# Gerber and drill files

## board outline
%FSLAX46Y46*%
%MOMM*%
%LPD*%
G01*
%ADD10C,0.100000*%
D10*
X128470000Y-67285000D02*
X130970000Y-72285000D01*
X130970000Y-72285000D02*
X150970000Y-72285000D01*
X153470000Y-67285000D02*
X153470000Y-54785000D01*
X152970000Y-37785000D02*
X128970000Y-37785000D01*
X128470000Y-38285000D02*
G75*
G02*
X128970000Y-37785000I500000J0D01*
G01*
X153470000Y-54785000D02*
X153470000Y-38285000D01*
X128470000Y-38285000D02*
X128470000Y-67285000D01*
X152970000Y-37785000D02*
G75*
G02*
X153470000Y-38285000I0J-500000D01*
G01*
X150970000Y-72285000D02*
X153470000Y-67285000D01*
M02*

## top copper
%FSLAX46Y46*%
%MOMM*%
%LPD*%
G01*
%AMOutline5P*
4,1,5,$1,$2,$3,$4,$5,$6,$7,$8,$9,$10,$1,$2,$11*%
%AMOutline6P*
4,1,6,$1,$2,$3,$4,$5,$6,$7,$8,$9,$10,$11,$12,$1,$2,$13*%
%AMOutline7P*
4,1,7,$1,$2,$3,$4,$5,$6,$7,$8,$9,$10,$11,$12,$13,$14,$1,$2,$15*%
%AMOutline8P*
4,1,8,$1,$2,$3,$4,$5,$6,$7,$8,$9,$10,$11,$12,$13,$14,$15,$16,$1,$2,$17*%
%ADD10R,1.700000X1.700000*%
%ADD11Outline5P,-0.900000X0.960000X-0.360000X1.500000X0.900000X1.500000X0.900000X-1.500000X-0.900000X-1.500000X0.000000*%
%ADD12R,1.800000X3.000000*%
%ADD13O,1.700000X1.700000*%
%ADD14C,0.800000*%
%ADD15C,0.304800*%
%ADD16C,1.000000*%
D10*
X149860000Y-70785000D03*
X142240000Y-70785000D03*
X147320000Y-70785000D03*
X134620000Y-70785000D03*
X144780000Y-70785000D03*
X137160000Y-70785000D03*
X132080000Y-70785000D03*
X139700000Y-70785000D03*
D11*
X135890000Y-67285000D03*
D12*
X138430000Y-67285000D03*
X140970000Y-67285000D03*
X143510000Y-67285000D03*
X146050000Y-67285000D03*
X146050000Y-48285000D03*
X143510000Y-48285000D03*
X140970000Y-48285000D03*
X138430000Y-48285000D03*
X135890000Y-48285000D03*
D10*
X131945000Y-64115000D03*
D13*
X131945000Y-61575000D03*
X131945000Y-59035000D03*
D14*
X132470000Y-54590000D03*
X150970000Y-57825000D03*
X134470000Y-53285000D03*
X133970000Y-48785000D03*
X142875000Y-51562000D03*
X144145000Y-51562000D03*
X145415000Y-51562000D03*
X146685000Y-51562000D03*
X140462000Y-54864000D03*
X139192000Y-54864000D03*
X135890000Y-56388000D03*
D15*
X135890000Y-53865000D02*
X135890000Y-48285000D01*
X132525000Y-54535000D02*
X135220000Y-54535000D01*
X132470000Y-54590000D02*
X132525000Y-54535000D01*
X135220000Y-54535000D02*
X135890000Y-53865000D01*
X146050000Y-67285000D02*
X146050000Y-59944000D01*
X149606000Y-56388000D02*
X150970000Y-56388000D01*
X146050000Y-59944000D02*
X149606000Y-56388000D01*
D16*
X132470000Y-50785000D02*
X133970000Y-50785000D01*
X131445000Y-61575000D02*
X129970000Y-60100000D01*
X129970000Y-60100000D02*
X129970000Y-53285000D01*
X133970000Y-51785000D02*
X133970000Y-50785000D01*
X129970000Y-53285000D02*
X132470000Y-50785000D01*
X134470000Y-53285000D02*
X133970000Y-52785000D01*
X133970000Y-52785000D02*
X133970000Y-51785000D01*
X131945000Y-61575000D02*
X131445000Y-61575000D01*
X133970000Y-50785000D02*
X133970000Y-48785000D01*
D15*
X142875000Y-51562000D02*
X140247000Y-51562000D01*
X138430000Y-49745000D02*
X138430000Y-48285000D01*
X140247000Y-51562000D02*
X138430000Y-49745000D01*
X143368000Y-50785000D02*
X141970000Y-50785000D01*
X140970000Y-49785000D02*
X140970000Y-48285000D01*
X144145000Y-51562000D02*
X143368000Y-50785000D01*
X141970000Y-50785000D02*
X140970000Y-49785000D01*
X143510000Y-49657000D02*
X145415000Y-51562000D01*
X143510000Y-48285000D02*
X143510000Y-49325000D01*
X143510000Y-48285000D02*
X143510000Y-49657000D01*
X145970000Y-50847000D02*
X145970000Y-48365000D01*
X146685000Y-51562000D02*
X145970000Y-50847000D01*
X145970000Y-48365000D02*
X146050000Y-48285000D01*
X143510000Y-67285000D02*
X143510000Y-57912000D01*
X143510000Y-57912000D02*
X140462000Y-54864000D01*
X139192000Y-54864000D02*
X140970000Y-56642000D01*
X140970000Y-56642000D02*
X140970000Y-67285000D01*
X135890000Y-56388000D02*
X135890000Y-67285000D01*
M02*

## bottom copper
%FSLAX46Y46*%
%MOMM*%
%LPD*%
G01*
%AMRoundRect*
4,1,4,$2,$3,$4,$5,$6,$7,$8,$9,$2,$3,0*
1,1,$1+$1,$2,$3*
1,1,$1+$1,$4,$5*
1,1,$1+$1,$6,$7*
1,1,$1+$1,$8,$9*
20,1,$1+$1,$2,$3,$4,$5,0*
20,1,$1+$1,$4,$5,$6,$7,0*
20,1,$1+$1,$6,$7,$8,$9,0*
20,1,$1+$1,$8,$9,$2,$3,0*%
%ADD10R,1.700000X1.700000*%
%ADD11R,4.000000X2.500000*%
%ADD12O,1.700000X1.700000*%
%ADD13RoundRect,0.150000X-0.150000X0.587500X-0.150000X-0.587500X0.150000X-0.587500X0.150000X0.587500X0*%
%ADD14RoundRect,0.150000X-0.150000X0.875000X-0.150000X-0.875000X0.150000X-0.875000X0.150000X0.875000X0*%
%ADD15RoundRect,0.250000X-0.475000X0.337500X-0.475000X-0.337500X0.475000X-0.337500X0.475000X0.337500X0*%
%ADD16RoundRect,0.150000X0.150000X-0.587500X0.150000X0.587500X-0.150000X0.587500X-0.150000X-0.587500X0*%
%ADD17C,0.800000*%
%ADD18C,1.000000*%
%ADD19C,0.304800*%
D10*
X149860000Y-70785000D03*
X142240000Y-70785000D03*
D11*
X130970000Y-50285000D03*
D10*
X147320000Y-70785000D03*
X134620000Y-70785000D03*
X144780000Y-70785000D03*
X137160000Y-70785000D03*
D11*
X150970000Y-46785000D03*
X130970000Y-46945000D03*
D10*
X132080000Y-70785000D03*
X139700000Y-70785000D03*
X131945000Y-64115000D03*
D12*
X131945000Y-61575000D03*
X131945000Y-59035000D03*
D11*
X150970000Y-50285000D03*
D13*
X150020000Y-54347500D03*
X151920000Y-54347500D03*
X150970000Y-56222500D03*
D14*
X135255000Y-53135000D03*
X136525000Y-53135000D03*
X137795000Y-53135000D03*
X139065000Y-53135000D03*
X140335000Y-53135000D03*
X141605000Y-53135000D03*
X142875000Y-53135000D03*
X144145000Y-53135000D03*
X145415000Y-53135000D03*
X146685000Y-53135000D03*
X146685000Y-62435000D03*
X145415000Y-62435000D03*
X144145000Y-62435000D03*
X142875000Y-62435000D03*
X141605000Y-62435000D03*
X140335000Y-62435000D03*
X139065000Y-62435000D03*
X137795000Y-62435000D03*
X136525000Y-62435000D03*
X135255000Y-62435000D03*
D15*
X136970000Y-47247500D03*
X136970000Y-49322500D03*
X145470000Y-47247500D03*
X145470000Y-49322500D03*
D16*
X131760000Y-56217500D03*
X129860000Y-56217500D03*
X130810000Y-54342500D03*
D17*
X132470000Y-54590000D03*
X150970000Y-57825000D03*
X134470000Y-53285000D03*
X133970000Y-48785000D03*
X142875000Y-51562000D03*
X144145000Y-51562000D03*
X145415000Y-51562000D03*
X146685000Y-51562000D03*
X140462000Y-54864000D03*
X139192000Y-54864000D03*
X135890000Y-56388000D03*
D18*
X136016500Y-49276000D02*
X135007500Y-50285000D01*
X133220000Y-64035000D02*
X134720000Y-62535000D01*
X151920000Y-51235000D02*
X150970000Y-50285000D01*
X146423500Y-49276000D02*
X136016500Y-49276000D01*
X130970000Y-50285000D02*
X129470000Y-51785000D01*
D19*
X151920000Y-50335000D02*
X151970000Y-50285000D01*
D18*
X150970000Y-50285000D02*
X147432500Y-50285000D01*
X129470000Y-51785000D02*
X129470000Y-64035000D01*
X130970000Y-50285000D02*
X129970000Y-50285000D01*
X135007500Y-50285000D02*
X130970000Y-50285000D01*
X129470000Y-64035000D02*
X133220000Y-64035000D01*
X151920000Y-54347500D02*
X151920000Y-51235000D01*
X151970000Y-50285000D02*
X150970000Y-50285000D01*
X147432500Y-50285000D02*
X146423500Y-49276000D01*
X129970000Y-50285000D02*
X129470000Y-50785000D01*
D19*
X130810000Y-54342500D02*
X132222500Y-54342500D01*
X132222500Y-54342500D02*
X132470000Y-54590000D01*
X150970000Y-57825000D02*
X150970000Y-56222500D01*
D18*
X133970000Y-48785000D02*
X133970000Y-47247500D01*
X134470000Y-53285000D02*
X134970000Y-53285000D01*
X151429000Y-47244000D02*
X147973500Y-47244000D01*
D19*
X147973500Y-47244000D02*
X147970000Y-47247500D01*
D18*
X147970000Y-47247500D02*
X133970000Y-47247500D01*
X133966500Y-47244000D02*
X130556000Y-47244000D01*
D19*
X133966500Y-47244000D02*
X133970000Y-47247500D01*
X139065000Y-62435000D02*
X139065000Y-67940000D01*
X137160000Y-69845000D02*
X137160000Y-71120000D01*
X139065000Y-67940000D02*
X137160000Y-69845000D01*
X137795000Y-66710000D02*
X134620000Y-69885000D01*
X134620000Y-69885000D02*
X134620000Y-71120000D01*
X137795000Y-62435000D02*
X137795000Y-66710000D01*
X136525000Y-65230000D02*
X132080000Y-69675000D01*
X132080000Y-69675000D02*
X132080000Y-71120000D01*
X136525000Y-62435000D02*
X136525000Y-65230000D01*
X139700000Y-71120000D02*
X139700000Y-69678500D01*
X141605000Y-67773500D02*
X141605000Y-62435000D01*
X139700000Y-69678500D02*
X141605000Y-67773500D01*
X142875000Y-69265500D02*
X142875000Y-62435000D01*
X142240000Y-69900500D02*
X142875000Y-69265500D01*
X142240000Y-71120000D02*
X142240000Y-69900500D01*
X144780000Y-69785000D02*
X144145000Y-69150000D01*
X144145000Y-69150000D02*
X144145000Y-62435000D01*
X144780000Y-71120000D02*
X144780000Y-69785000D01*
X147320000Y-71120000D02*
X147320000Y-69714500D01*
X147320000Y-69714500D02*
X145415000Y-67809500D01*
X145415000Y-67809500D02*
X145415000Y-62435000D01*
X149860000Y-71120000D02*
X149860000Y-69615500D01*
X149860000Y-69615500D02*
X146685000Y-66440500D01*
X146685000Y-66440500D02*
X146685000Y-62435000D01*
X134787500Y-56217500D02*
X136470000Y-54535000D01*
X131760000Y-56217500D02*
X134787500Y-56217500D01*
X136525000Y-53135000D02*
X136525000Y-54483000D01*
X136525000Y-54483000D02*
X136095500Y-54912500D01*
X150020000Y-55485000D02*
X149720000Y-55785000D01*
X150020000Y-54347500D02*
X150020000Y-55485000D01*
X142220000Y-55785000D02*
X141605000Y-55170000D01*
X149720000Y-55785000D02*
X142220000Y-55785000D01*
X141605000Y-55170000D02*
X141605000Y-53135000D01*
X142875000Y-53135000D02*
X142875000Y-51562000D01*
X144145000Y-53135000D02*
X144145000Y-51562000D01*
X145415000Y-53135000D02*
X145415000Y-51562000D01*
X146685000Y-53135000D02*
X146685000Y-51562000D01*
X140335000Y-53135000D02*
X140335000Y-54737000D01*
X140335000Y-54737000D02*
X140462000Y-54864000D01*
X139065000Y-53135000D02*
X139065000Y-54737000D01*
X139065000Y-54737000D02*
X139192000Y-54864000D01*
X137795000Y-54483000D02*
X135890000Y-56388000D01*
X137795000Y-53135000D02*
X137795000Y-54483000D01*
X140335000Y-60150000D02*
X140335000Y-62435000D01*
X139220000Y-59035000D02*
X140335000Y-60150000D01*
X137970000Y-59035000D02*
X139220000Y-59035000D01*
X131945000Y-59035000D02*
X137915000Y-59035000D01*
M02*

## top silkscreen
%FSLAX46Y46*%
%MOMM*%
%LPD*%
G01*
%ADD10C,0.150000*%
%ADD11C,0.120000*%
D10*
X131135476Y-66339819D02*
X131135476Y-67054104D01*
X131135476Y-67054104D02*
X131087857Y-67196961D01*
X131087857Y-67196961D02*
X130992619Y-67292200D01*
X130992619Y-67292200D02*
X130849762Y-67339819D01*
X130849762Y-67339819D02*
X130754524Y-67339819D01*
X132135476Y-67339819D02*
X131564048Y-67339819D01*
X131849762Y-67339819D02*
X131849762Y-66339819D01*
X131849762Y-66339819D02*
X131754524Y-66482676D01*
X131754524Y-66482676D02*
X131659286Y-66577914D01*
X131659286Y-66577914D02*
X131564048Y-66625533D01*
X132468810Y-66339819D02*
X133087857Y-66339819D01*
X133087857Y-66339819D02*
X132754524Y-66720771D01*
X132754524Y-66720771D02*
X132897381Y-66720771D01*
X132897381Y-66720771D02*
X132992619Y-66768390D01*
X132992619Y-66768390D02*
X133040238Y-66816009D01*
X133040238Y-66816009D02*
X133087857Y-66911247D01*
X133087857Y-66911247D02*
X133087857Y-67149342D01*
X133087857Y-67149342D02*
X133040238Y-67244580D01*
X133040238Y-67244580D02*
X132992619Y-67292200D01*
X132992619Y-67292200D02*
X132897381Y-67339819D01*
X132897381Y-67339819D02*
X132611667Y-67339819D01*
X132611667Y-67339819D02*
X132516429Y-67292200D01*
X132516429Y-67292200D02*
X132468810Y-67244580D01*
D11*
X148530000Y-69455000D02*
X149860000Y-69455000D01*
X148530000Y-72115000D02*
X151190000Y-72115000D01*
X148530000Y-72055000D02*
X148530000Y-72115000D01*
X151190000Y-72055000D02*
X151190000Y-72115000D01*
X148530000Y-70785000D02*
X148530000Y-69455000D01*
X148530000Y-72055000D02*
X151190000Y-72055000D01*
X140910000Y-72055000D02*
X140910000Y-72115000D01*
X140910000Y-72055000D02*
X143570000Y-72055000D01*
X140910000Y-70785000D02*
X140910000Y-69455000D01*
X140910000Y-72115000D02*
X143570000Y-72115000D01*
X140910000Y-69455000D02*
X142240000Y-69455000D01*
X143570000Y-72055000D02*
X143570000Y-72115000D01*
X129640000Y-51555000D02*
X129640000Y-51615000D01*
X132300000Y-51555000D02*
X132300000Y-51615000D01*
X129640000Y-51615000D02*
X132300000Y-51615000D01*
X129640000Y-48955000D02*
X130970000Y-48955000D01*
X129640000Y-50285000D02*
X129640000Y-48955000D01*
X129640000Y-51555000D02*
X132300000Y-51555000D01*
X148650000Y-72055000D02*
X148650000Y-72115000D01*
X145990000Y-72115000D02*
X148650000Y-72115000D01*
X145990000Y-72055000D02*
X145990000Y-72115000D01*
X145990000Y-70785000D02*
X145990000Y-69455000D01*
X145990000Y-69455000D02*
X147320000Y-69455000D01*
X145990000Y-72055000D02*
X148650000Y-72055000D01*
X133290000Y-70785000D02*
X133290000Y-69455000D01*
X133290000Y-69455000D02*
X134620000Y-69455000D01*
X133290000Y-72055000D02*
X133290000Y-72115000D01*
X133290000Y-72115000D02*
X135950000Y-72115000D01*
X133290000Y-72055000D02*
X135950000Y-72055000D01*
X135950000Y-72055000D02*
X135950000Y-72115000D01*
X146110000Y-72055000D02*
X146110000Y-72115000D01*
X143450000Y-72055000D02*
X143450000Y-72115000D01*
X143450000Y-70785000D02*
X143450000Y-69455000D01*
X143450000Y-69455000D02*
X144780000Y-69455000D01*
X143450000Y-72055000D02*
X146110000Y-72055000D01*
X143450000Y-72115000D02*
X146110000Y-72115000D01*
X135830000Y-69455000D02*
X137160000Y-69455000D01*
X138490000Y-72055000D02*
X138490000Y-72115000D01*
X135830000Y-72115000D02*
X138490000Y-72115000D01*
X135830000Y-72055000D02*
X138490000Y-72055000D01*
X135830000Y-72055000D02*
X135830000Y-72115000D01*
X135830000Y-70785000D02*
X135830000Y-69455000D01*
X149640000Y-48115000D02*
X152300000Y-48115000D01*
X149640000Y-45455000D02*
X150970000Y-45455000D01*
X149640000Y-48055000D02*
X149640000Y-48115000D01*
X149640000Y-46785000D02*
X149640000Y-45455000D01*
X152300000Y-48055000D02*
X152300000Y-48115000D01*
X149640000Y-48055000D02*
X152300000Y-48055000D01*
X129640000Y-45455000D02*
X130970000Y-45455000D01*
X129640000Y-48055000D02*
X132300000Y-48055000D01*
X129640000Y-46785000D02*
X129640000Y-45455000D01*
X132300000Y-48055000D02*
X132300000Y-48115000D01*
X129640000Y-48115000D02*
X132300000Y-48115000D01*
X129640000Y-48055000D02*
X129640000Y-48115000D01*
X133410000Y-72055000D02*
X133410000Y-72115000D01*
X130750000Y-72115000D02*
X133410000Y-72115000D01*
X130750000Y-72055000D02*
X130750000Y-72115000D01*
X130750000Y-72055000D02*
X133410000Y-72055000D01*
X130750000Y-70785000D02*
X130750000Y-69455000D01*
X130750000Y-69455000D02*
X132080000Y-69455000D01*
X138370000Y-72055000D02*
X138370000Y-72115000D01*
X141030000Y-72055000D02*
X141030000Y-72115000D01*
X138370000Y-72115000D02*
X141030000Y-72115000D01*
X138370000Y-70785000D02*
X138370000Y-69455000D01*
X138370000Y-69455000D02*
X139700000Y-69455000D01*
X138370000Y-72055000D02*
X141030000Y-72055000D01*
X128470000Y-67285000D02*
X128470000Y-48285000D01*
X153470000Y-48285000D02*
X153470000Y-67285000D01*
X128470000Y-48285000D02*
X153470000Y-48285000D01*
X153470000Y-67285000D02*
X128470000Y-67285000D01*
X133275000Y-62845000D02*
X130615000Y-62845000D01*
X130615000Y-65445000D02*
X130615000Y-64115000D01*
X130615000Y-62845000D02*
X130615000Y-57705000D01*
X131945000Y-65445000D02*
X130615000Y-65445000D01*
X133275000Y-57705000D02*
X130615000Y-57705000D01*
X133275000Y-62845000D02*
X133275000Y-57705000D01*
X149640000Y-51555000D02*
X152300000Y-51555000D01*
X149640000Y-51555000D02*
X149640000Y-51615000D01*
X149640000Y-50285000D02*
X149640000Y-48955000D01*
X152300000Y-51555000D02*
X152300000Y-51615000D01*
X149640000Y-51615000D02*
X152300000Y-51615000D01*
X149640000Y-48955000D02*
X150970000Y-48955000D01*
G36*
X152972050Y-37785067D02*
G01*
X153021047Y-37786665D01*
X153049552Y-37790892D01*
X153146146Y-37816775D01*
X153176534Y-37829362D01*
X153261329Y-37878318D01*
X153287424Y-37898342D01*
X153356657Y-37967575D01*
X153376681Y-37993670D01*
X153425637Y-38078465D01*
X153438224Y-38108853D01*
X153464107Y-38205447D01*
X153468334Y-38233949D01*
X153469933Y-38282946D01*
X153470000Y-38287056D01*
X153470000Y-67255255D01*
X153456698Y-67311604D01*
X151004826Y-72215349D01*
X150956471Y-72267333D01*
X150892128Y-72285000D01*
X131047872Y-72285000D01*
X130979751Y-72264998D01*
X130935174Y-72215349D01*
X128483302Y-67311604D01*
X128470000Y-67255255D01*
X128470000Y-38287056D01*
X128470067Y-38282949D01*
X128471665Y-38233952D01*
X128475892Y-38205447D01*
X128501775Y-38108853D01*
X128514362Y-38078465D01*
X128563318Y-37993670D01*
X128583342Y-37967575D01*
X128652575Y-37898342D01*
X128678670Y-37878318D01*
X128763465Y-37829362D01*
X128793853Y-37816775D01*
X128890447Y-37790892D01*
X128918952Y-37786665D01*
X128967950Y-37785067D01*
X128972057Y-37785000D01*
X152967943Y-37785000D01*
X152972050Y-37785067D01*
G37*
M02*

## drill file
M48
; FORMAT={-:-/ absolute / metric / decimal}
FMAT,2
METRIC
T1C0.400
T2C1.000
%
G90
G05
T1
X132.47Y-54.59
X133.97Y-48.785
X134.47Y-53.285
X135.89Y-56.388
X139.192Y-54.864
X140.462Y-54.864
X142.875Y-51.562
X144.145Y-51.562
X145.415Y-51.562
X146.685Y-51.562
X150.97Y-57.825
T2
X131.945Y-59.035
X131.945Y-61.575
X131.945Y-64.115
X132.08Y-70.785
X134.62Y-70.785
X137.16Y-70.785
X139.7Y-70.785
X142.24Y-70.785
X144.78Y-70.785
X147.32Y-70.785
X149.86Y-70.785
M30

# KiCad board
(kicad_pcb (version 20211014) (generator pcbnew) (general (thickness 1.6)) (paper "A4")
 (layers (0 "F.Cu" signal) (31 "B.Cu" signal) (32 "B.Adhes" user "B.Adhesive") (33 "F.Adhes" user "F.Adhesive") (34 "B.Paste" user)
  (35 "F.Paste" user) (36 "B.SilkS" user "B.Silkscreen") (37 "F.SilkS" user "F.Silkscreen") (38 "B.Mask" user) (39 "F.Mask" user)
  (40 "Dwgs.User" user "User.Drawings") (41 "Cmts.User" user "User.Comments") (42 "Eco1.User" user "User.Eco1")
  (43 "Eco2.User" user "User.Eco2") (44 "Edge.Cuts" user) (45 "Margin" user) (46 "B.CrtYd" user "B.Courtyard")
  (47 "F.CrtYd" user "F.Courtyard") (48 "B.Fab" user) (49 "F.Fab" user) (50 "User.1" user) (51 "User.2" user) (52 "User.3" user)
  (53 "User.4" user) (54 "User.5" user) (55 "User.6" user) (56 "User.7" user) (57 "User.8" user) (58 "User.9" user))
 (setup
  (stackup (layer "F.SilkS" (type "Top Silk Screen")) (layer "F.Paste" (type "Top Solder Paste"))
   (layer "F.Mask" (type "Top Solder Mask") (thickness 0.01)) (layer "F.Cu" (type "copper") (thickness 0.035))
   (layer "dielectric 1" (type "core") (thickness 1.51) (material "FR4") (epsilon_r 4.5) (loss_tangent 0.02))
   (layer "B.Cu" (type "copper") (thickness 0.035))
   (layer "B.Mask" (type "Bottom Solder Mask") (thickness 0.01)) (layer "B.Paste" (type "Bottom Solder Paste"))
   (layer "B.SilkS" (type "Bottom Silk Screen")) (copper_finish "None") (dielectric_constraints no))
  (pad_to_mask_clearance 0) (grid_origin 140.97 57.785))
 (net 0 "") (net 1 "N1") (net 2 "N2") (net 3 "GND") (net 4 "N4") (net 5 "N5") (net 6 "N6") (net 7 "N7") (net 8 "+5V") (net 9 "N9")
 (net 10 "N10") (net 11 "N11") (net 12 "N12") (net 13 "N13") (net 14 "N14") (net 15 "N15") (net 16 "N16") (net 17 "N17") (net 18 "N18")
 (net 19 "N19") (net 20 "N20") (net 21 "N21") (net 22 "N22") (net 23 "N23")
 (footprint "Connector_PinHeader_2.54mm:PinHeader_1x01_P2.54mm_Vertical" (layer "F.Cu") (at 149.86 70.785)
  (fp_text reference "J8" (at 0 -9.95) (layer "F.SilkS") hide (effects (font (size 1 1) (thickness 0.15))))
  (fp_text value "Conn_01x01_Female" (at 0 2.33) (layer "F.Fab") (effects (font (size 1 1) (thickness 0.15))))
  (fp_line (start -1.33 -1.33) (end 0 -1.33) (layer "F.SilkS") (width 0.12))
  (fp_line (start -1.33 1.33) (end 1.33 1.33) (layer "F.SilkS") (width 0.12))
  (fp_line (start -1.33 1.27) (end -1.33 1.33) (layer "F.SilkS") (width 0.12))
  (fp_line (start 1.33 1.27) (end 1.33 1.33) (layer "F.SilkS") (width 0.12))
  (fp_line (start -1.33 0) (end -1.33 -1.33) (layer "F.SilkS") (width 0.12))
  (fp_line (start -1.33 1.27) (end 1.33 1.27) (layer "F.SilkS") (width 0.12))
  (pad "1" thru_hole rect (at 0 0) (size 1.7 1.7) (drill 1) (layers *.Cu *.Mask) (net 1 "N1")))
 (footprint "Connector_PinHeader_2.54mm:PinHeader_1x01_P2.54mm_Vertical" (layer "F.Cu") (at 142.24 70.785)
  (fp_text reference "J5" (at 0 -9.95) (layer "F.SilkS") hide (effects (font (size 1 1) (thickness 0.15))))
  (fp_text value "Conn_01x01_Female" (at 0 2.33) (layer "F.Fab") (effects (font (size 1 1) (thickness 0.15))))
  (fp_line (start -1.33 1.27) (end -1.33 1.33) (layer "F.SilkS") (width 0.12))
  (fp_line (start -1.33 1.27) (end 1.33 1.27) (layer "F.SilkS") (width 0.12))
  (fp_line (start -1.33 0) (end -1.33 -1.33) (layer "F.SilkS") (width 0.12))
  (fp_line (start -1.33 1.33) (end 1.33 1.33) (layer "F.SilkS") (width 0.12))
  (fp_line (start -1.33 -1.33) (end 0 -1.33) (layer "F.SilkS") (width 0.12))
  (fp_line (start 1.33 1.27) (end 1.33 1.33) (layer "F.SilkS") (width 0.12))
  (pad "1" thru_hole rect (at 0 0) (size 1.7 1.7) (drill 1) (layers *.Cu *.Mask) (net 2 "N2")))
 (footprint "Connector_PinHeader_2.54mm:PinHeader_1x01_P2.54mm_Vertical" (layer "F.Cu") (at 130.97 50.285)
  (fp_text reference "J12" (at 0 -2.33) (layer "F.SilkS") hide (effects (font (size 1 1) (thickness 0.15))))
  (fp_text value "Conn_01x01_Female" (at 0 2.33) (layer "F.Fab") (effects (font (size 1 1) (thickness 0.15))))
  (fp_line (start -1.33 1.27) (end -1.33 1.33) (layer "F.SilkS") (width 0.12))
  (fp_line (start 1.33 1.27) (end 1.33 1.33) (layer "F.SilkS") (width 0.12))
  (fp_line (start -1.33 1.33) (end 1.33 1.33) (layer "F.SilkS") (width 0.12))
  (fp_line (start -1.33 -1.33) (end 0 -1.33) (layer "F.SilkS") (width 0.12))
  (fp_line (start -1.33 0) (end -1.33 -1.33) (layer "F.SilkS") (width 0.12))
  (fp_line (start -1.33 1.27) (end 1.33 1.27) (layer "F.SilkS") (width 0.12))
  (pad "1" smd rect (at 0 0) (size 4 2.5) (layers "B.Cu" "B.Mask") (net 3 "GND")))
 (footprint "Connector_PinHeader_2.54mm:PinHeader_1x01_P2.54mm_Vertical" (layer "F.Cu") (at 147.32 70.785)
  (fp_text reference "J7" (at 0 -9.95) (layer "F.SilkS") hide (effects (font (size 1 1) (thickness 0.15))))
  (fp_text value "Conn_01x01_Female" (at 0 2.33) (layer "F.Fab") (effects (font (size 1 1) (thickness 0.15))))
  (fp_line (start 1.33 1.27) (end 1.33 1.33) (layer "F.SilkS") (width 0.12))
  (fp_line (start -1.33 1.33) (end 1.33 1.33) (layer "F.SilkS") (width 0.12))
  (fp_line (start -1.33 1.27) (end -1.33 1.33) (layer "F.SilkS") (width 0.12))
  (fp_line (start -1.33 0) (end -1.33 -1.33) (layer "F.SilkS") (width 0.12))
  (fp_line (start -1.33 -1.33) (end 0 -1.33) (layer "F.SilkS") (width 0.12))
  (fp_line (start -1.33 1.27) (end 1.33 1.27) (layer "F.SilkS") (width 0.12))
  (pad "1" thru_hole rect (at 0 0) (size 1.7 1.7) (drill 1) (layers *.Cu *.Mask) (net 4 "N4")))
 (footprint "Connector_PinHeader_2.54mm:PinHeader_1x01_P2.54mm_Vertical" (layer "F.Cu") (at 134.62 70.785)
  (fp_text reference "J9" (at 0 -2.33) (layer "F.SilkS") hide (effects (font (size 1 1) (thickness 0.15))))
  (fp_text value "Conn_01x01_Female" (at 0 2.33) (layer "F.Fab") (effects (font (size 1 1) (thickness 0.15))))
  (fp_line (start -1.33 0) (end -1.33 -1.33) (layer "F.SilkS") (width 0.12))
  (fp_line (start -1.33 -1.33) (end 0 -1.33) (layer "F.SilkS") (width 0.12))
  (fp_line (start -1.33 1.27) (end -1.33 1.33) (layer "F.SilkS") (width 0.12))
  (fp_line (start -1.33 1.33) (end 1.33 1.33) (layer "F.SilkS") (width 0.12))
  (fp_line (start -1.33 1.27) (end 1.33 1.27) (layer "F.SilkS") (width 0.12))
  (fp_line (start 1.33 1.27) (end 1.33 1.33) (layer "F.SilkS") (width 0.12))
  (pad "1" thru_hole rect (at 0 0) (size 1.7 1.7) (drill 1) (layers *.Cu *.Mask) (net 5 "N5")))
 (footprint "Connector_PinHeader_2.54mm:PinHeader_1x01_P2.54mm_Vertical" (layer "F.Cu") (at 144.78 70.785)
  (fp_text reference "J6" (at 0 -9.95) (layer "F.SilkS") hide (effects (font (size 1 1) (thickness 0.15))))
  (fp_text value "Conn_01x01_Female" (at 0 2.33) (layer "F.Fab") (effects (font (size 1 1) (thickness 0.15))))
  (fp_line (start 1.33 1.27) (end 1.33 1.33) (layer "F.SilkS") (width 0.12))
  (fp_line (start -1.33 1.27) (end -1.33 1.33) (layer "F.SilkS") (width 0.12))
  (fp_line (start -1.33 0) (end -1.33 -1.33) (layer "F.SilkS") (width 0.12))
  (fp_line (start -1.33 -1.33) (end 0 -1.33) (layer "F.SilkS") (width 0.12))
  (fp_line (start -1.33 1.27) (end 1.33 1.27) (layer "F.SilkS") (width 0.12))
  (fp_line (start -1.33 1.33) (end 1.33 1.33) (layer "F.SilkS") (width 0.12))
  (pad "1" thru_hole rect (at 0 0) (size 1.7 1.7) (drill 1) (layers *.Cu *.Mask) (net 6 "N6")))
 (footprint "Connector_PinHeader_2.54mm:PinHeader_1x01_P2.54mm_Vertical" (layer "F.Cu") (at 137.16 70.785)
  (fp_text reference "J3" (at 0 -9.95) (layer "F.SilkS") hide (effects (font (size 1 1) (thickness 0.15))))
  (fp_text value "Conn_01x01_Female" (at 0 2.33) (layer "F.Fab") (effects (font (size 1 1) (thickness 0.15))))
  (fp_line (start -1.33 -1.33) (end 0 -1.33) (layer "F.SilkS") (width 0.12))
  (fp_line (start 1.33 1.27) (end 1.33 1.33) (layer "F.SilkS") (width 0.12))
  (fp_line (start -1.33 1.33) (end 1.33 1.33) (layer "F.SilkS") (width 0.12))
  (fp_line (start -1.33 1.27) (end 1.33 1.27) (layer "F.SilkS") (width 0.12))
  (fp_line (start -1.33 1.27) (end -1.33 1.33) (layer "F.SilkS") (width 0.12))
  (fp_line (start -1.33 0) (end -1.33 -1.33) (layer "F.SilkS") (width 0.12))
  (pad "1" thru_hole rect (at 0 0) (size 1.7 1.7) (drill 1) (layers *.Cu *.Mask) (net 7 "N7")))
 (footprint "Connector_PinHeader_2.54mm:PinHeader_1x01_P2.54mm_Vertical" (layer "F.Cu") (at 150.97 46.785)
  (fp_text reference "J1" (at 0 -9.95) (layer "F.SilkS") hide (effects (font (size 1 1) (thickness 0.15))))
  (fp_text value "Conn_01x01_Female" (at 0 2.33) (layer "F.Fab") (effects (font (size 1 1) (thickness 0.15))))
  (fp_line (start -1.33 1.33) (end 1.33 1.33) (layer "F.SilkS") (width 0.12))
  (fp_line (start -1.33 -1.33) (end 0 -1.33) (layer "F.SilkS") (width 0.12))
  (fp_line (start -1.33 1.27) (end -1.33 1.33) (layer "F.SilkS") (width 0.12))
  (fp_line (start -1.33 0) (end -1.33 -1.33) (layer "F.SilkS") (width 0.12))
  (fp_line (start 1.33 1.27) (end 1.33 1.33) (layer "F.SilkS") (width 0.12))
  (fp_line (start -1.33 1.27) (end 1.33 1.27) (layer "F.SilkS") (width 0.12))
  (pad "1" smd rect (at 0 0) (size 4 2.5) (layers "B.Cu" "B.Mask") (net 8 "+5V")))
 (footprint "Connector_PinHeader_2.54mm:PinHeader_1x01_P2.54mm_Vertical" (layer "F.Cu") (at 130.97 46.785)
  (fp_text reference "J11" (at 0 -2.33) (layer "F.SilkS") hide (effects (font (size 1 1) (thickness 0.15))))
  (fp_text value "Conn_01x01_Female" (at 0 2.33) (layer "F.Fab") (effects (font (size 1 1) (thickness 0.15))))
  (fp_line (start -1.33 -1.33) (end 0 -1.33) (layer "F.SilkS") (width 0.12))
  (fp_line (start -1.33 1.27) (end 1.33 1.27) (layer "F.SilkS") (width 0.12))
  (fp_line (start -1.33 0) (end -1.33 -1.33) (layer "F.SilkS") (width 0.12))
  (fp_line (start 1.33 1.27) (end 1.33 1.33) (layer "F.SilkS") (width 0.12))
  (fp_line (start -1.33 1.33) (end 1.33 1.33) (layer "F.SilkS") (width 0.12))
  (fp_line (start -1.33 1.27) (end -1.33 1.33) (layer "F.SilkS") (width 0.12))
  (pad "1" smd rect (at 0 0.16) (size 4 2.5) (layers "B.Cu" "B.Mask") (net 8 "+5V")))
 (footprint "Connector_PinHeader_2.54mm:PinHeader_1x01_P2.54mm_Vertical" (layer "F.Cu") (at 132.08 70.785)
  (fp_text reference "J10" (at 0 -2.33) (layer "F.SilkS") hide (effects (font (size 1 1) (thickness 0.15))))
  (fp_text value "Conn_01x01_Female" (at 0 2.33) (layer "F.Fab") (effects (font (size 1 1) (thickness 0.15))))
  (fp_line (start 1.33 1.27) (end 1.33 1.33) (layer "F.SilkS") (width 0.12))
  (fp_line (start -1.33 1.33) (end 1.33 1.33) (layer "F.SilkS") (width 0.12))
  (fp_line (start -1.33 1.27) (end -1.33 1.33) (layer "F.SilkS") (width 0.12))
  (fp_line (start -1.33 1.27) (end 1.33 1.27) (layer "F.SilkS") (width 0.12))
  (fp_line (start -1.33 0) (end -1.33 -1.33) (layer "F.SilkS") (width 0.12))
  (fp_line (start -1.33 -1.33) (end 0 -1.33) (layer "F.SilkS") (width 0.12))
  (pad "1" thru_hole rect (at 0 0) (size 1.7 1.7) (drill 1) (layers *.Cu *.Mask) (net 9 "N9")))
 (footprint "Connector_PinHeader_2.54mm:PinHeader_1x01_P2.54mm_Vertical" (layer "F.Cu") (at 139.7 70.785)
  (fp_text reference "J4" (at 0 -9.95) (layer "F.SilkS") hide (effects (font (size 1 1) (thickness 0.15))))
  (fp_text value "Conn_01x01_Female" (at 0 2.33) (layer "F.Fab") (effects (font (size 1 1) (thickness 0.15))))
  (fp_line (start -1.33 1.27) (end -1.33 1.33) (layer "F.SilkS") (width 0.12))
  (fp_line (start 1.33 1.27) (end 1.33 1.33) (layer "F.SilkS") (width 0.12))
  (fp_line (start -1.33 1.33) (end 1.33 1.33) (layer "F.SilkS") (width 0.12))
  (fp_line (start -1.33 0) (end -1.33 -1.33) (layer "F.SilkS") (width 0.12))
  (fp_line (start -1.33 -1.33) (end 0 -1.33) (layer "F.SilkS") (width 0.12))
  (fp_line (start -1.33 1.27) (end 1.33 1.27) (layer "F.SilkS") (width 0.12))
  (pad "1" thru_hole rect (at 0 0) (size 1.7 1.7) (drill 1) (layers *.Cu *.Mask) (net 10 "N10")))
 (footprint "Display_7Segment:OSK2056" (layer "F.Cu") (at 140.97 57.785)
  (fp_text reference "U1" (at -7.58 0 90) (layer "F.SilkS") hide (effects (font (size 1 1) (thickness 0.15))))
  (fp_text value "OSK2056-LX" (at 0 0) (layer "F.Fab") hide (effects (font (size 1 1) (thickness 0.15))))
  (fp_line (start -12.5 9.5) (end -12.5 -9.5) (layer "F.SilkS") (width 0.12))
  (fp_line (start 12.5 -9.5) (end 12.5 9.5) (layer "F.SilkS") (width 0.12))
  (fp_line (start -12.5 -9.5) (end 12.5 -9.5) (layer "F.SilkS") (width 0.12))
  (fp_line (start 12.5 9.5) (end -12.5 9.5) (layer "F.SilkS") (width 0.12))
  (pad "1" smd roundrect (at -5.08 9.5) (size 1.8 3) (layers "F.Cu" "F.Paste" "F.Mask") (roundrect_rratio 0) (chamfer_ratio 0.3)
   (chamfer top_left) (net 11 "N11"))
  (pad "2" smd rect (at -2.54 9.5) (size 1.8 3) (layers "F.Cu" "F.Paste" "F.Mask") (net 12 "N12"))
  (pad "3" smd rect (at 0 9.5) (size 1.8 3) (layers "F.Cu" "F.Paste" "F.Mask") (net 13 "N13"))
  (pad "4" smd rect (at 2.54 9.5) (size 1.8 3) (layers "F.Cu" "F.Paste" "F.Mask") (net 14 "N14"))
  (pad "5" smd rect (at 5.08 9.5) (size 1.8 3) (layers "F.Cu" "F.Paste" "F.Mask") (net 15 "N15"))
  (pad "6" smd rect (at 5.08 -9.5) (size 1.8 3) (layers "F.Cu" "F.Paste" "F.Mask") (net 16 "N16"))
  (pad "7" smd rect (at 2.54 -9.5) (size 1.8 3) (layers "F.Cu" "F.Paste" "F.Mask") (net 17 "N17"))
  (pad "8" smd rect (at 0 -9.5) (size 1.8 3) (layers "F.Cu" "F.Paste" "F.Mask") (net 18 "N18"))
  (pad "9" smd rect (at -2.54 -9.5) (size 1.8 3) (layers "F.Cu" "F.Paste" "F.Mask") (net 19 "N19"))
  (pad "10" smd rect (at -5.08 -9.5) (size 1.8 3) (layers "F.Cu" "F.Paste" "F.Mask") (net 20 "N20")))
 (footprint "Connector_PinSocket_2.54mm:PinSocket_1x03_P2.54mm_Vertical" (layer "F.Cu") (at 131.945 64.115 180)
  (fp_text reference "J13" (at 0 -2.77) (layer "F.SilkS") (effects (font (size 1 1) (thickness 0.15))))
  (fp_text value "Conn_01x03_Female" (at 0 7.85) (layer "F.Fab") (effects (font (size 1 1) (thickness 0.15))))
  (fp_line (start -1.33 1.27) (end 1.33 1.27) (layer "F.SilkS") (width 0.12))
  (fp_line (start 1.33 -1.33) (end 1.33 0) (layer "F.SilkS") (width 0.12))
  (fp_line (start 1.33 1.27) (end 1.33 6.41) (layer "F.SilkS") (width 0.12))
  (fp_line (start 0 -1.33) (end 1.33 -1.33) (layer "F.SilkS") (width 0.12))
  (fp_line (start -1.33 6.41) (end 1.33 6.41) (layer "F.SilkS") (width 0.12))
  (fp_line (start -1.33 1.27) (end -1.33 6.41) (layer "F.SilkS") (width 0.12))
  (pad "1" thru_hole rect (at 0 0 180) (size 1.7 1.7) (drill 1) (layers *.Cu *.Mask) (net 3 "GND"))
  (pad "2" thru_hole oval (at 0 2.54 180) (size 1.7 1.7) (drill 1) (layers *.Cu *.Mask) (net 8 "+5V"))
  (pad "3" thru_hole oval (at 0 5.08 180) (size 1.7 1.7) (drill 1) (layers *.Cu *.Mask) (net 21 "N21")))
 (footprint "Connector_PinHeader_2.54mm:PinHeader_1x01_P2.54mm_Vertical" (layer "F.Cu") (at 150.97 50.285)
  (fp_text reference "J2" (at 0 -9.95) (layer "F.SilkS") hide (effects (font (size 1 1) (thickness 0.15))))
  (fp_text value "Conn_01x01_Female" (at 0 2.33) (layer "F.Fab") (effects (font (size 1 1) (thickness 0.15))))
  (fp_line (start -1.33 1.27) (end 1.33 1.27) (layer "F.SilkS") (width 0.12))
  (fp_line (start -1.33 1.27) (end -1.33 1.33) (layer "F.SilkS") (width 0.12))
  (fp_line (start -1.33 0) (end -1.33 -1.33) (layer "F.SilkS") (width 0.12))
  (fp_line (start 1.33 1.27) (end 1.33 1.33) (layer "F.SilkS") (width 0.12))
  (fp_line (start -1.33 1.33) (end 1.33 1.33) (layer "F.SilkS") (width 0.12))
  (fp_line (start -1.33 -1.33) (end 0 -1.33) (layer "F.SilkS") (width 0.12))
  (pad "1" smd rect (at 0 0) (size 4 2.5) (layers "B.Cu" "B.Mask") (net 3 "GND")))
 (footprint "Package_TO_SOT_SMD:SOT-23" (layer "B.Cu") (at 150.97 55.285 -90)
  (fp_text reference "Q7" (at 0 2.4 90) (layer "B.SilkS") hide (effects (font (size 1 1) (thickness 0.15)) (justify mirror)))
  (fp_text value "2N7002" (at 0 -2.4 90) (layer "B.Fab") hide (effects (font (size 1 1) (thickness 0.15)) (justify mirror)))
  (pad "1" smd roundrect (at -0.9375 0.95 270) (size 1.475 0.6) (layers "B.Cu" "B.Paste" "B.Mask") (roundrect_rratio 0.25) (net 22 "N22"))
  (pad "2" smd roundrect (at -0.9375 -0.95 270) (size 1.475 0.6) (layers "B.Cu" "B.Paste" "B.Mask") (roundrect_rratio 0.25) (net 3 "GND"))
  (pad "3" smd roundrect (at 0.9375 0 270) (size 1.475 0.6) (layers "B.Cu" "B.Paste" "B.Mask") (roundrect_rratio 0.25) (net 15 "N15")))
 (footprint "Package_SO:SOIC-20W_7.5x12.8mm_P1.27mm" (layer "B.Cu") (at 140.97 57.785 -90)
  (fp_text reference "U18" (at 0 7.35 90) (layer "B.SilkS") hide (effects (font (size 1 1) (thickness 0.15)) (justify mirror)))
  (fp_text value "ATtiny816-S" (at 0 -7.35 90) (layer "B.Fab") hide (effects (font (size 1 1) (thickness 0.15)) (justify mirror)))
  (pad "1" smd roundrect (at -4.65 5.715 270) (size 2.05 0.6) (layers "B.Cu" "B.Paste" "B.Mask") (roundrect_rratio 0.25) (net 8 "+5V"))
  (pad "2" smd roundrect (at -4.65 4.445 270) (size 2.05 0.6) (layers "B.Cu" "B.Paste" "B.Mask") (roundrect_rratio 0.25) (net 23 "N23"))
  (pad "3" smd roundrect (at -4.65 3.175 270) (size 2.05 0.6) (layers "B.Cu" "B.Paste" "B.Mask") (roundrect_rratio 0.25) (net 11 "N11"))
  (pad "4" smd roundrect (at -4.65 1.905 270) (size 2.05 0.6) (layers "B.Cu" "B.Paste" "B.Mask") (roundrect_rratio 0.25) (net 13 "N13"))
  (pad "5" smd roundrect (at -4.65 0.635 270) (size 2.05 0.6) (layers "B.Cu" "B.Paste" "B.Mask") (roundrect_rratio 0.25) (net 14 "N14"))
  (pad "6" smd roundrect (at -4.65 -0.635 270) (size 2.05 0.6) (layers "B.Cu" "B.Paste" "B.Mask") (roundrect_rratio 0.25) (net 22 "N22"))
  (pad "7" smd roundrect (at -4.65 -1.905 270) (size 2.05 0.6) (layers "B.Cu" "B.Paste" "B.Mask") (roundrect_rratio 0.25) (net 19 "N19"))
  (pad "8" smd roundrect (at -4.65 -3.175 270) (size 2.05 0.6) (layers "B.Cu" "B.Paste" "B.Mask") (roundrect_rratio 0.25) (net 18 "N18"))
  (pad "9" smd roundrect (at -4.65 -4.445 270) (size 2.05 0.6) (layers "B.Cu" "B.Paste" "B.Mask") (roundrect_rratio 0.25) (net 17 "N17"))
  (pad "10" smd roundrect (at -4.65 -5.715 270) (size 2.05 0.6) (layers "B.Cu" "B.Paste" "B.Mask") (roundrect_rratio 0.25) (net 16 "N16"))
  (pad "11" smd roundrect (at 4.65 -5.715 270) (size 2.05 0.6) (layers "B.Cu" "B.Paste" "B.Mask") (roundrect_rratio 0.25) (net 1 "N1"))
  (pad "12" smd roundrect (at 4.65 -4.445 270) (size 2.05 0.6) (layers "B.Cu" "B.Paste" "B.Mask") (roundrect_rratio 0.25) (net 4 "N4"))
  (pad "13" smd roundrect (at 4.65 -3.175 270) (size 2.05 0.6) (layers "B.Cu" "B.Paste" "B.Mask") (roundrect_rratio 0.25) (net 6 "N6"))
  (pad "14" smd roundrect (at 4.65 -1.905 270) (size 2.05 0.6) (layers "B.Cu" "B.Paste" "B.Mask") (roundrect_rratio 0.25) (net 2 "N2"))
  (pad "15" smd roundrect (at 4.65 -0.635 270) (size 2.05 0.6) (layers "B.Cu" "B.Paste" "B.Mask") (roundrect_rratio 0.25) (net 10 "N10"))
  (pad "16" smd roundrect (at 4.65 0.635 270) (size 2.05 0.6) (layers "B.Cu" "B.Paste" "B.Mask") (roundrect_rratio 0.25) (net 21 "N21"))
  (pad "17" smd roundrect (at 4.65 1.905 270) (size 2.05 0.6) (layers "B.Cu" "B.Paste" "B.Mask") (roundrect_rratio 0.25) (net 7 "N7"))
  (pad "18" smd roundrect (at 4.65 3.175 270) (size 2.05 0.6) (layers "B.Cu" "B.Paste" "B.Mask") (roundrect_rratio 0.25) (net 5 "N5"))
  (pad "19" smd roundrect (at 4.65 4.445 270) (size 2.05 0.6) (layers "B.Cu" "B.Paste" "B.Mask") (roundrect_rratio 0.25) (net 9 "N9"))
  (pad "20" smd roundrect (at 4.65 5.715 270) (size 2.05 0.6) (layers "B.Cu" "B.Paste" "B.Mask") (roundrect_rratio 0.25) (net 3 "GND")))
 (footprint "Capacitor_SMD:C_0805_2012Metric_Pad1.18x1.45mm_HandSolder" (layer "B.Cu") (at 136.97 48.285 -90)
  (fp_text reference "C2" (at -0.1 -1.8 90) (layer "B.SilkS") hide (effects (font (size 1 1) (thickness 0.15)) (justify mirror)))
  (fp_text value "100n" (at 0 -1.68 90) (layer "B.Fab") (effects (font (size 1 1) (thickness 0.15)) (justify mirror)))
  (pad "1" smd roundrect (at -1.0375 0 270) (size 1.175 1.45) (layers "B.Cu" "B.Paste" "B.Mask") (roundrect_rratio 0.212766) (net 8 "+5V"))
  (pad "2" smd roundrect (at 1.0375 0 270) (size 1.175 1.45) (layers "B.Cu" "B.Paste" "B.Mask") (roundrect_rratio 0.212766) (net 3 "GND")))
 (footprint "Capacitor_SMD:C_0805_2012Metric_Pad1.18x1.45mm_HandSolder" (layer "B.Cu") (at 145.47 48.285 -90)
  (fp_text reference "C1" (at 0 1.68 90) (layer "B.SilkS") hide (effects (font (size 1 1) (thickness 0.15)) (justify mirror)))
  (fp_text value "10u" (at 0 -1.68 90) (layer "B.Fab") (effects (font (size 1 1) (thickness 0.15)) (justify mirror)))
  (pad "1" smd roundrect (at -1.0375 0 270) (size 1.175 1.45) (layers "B.Cu" "B.Paste" "B.Mask") (roundrect_rratio 0.212766) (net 8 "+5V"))
  (pad "2" smd roundrect (at 1.0375 0 270) (size 1.175 1.45) (layers "B.Cu" "B.Paste" "B.Mask") (roundrect_rratio 0.212766) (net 3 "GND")))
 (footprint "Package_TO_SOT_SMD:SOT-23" (layer "B.Cu") (at 130.81 55.28 90)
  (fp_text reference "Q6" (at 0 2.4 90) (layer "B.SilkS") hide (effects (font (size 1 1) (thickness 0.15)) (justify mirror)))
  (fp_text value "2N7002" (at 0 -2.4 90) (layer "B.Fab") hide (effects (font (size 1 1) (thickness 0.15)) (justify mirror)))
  (pad "1" smd roundrect (at -0.9375 0.95 90) (size 1.475 0.6) (layers "B.Cu" "B.Paste" "B.Mask") (roundrect_rratio 0.25) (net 23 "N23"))
  (pad "2" smd roundrect (at -0.9375 -0.95 90) (size 1.475 0.6) (layers "B.Cu" "B.Paste" "B.Mask") (roundrect_rratio 0.25) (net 3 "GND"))
  (pad "3" smd roundrect (at 0.9375 0 90) (size 1.475 0.6) (layers "B.Cu" "B.Paste" "B.Mask") (roundrect_rratio 0.25) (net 20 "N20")))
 (gr_line (start 128.47 67.285) (end 130.97 72.285) (layer "Edge.Cuts") (width 0.1))
 (gr_line (start 130.97 72.285) (end 150.97 72.285) (layer "Edge.Cuts") (width 0.1))
 (gr_line (start 153.47 67.285) (end 153.47 54.785) (layer "Edge.Cuts") (width 0.1))
 (gr_line (start 152.97 37.785) (end 128.97 37.785) (layer "Edge.Cuts") (width 0.1))
 (gr_arc (start 128.47 38.285) (mid 128.616447 37.931447) (end 128.97 37.785) (layer "Edge.Cuts") (width 0.1))
 (gr_line (start 153.47 54.785) (end 153.47 38.285) (layer "Edge.Cuts") (width 0.1))
 (gr_line (start 128.47 38.285) (end 128.47 67.285) (layer "Edge.Cuts") (width 0.1))
 (gr_arc (start 152.97 37.785) (mid 153.323553 37.931447) (end 153.47 38.285) (layer "Edge.Cuts") (width 0.1))
 (gr_line (start 150.97 72.285) (end 153.47 67.285) (layer "Edge.Cuts") (width 0.1))
 (segment (start 136.0165 49.276) (end 135.0075 50.285) (width 1) (layer "B.Cu") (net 3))
 (segment (start 133.22 64.035) (end 134.72 62.535) (width 1) (layer "B.Cu") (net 3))
 (segment (start 151.92 51.235) (end 150.97 50.285) (width 1) (layer "B.Cu") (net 3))
 (segment (start 146.4235 49.276) (end 136.0165 49.276) (width 1) (layer "B.Cu") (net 3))
 (segment (start 130.97 50.285) (end 129.47 51.785) (width 1) (layer "B.Cu") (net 3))
 (segment (start 151.92 50.335) (end 151.97 50.285) (width 0.3048) (layer "B.Cu") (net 3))
 (segment (start 150.97 50.285) (end 147.4325 50.285) (width 1) (layer "B.Cu") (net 3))
 (segment (start 129.47 51.785) (end 129.47 64.035) (width 1) (layer "B.Cu") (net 3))
 (segment (start 130.97 50.285) (end 129.97 50.285) (width 1) (layer "B.Cu") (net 3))
 (segment (start 135.0075 50.285) (end 130.97 50.285) (width 1) (layer "B.Cu") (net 3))
 (segment (start 129.47 64.035) (end 133.22 64.035) (width 1) (layer "B.Cu") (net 3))
 (segment (start 151.92 54.3475) (end 151.92 51.235) (width 1) (layer "B.Cu") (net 3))
 (segment (start 151.97 50.285) (end 150.97 50.285) (width 1) (layer "B.Cu") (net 3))
 (segment (start 147.4325 50.285) (end 146.4235 49.276) (width 1) (layer "B.Cu") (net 3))
 (segment (start 129.97 50.285) (end 129.47 50.785) (width 1) (layer "B.Cu") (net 3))
 (segment (start 135.89 53.865) (end 135.89 48.285) (width 0.3048) (layer "F.Cu") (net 20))
 (segment (start 132.525 54.535) (end 135.22 54.535) (width 0.3048) (layer "F.Cu") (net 20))
 (segment (start 132.47 54.59) (end 132.525 54.535) (width 0.3048) (layer "F.Cu") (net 20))
 (segment (start 135.22 54.535) (end 135.89 53.865) (width 0.3048) (layer "F.Cu") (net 20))
 (via (at 132.47 54.59) (size 0.8) (drill 0.4) (layers "F.Cu" "B.Cu") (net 20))
 (segment (start 130.81 54.3425) (end 132.2225 54.3425) (width 0.3048) (layer "B.Cu") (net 20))
 (segment (start 132.2225 54.3425) (end 132.47 54.59) (width 0.3048) (layer "B.Cu") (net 20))
 (segment (start 146.05 67.285) (end 146.05 59.944) (width 0.3048) (layer "F.Cu") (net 15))
 (segment (start 149.606 56.388) (end 150.97 56.388) (width 0.3048) (layer "F.Cu") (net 15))
 (segment (start 146.05 59.944) (end 149.606 56.388) (width 0.3048) (layer "F.Cu") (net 15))
 (via (at 150.97 57.825) (size 0.8) (drill 0.4) (layers "F.Cu" "B.Cu") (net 15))
 (segment (start 150.97 57.825) (end 150.97 56.2225) (width 0.3048) (layer "B.Cu") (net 15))
 (segment (start 132.47 50.785) (end 133.97 50.785) (width 1) (layer "F.Cu") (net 8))
 (segment (start 131.445 61.575) (end 129.97 60.1) (width 1) (layer "F.Cu") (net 8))
 (segment (start 129.97 60.1) (end 129.97 53.285) (width 1) (layer "F.Cu") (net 8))
 (segment (start 133.97 51.785) (end 133.97 50.785) (width 1) (layer "F.Cu") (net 8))
 (segment (start 129.97 53.285) (end 132.47 50.785) (width 1) (layer "F.Cu") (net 8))
 (segment (start 134.47 53.285) (end 133.97 52.785) (width 1) (layer "F.Cu") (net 8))
 (segment (start 133.97 52.785) (end 133.97 51.785) (width 1) (layer "F.Cu") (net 8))
 (segment (start 131.945 61.575) (end 131.445 61.575) (width 1) (layer "F.Cu") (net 8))
 (segment (start 133.97 50.785) (end 133.97 48.785) (width 1) (layer "F.Cu") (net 8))
 (via (at 134.47 53.285) (size 0.8) (drill 0.4) (layers "F.Cu" "B.Cu") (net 8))
 (via (at 133.97 48.785) (size 0.8) (drill 0.4) (layers "F.Cu" "B.Cu") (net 8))
 (segment (start 133.97 48.785) (end 133.97 47.2475) (width 1) (layer "B.Cu") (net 8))
 (segment (start 134.47 53.285) (end 134.97 53.285) (width 1) (layer "B.Cu") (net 8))
 (segment (start 151.429 47.244) (end 147.9735 47.244) (width 1) (layer "B.Cu") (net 8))
 (segment (start 147.9735 47.244) (end 147.97 47.2475) (width 0.3048) (layer "B.Cu") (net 8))
 (segment (start 147.97 47.2475) (end 133.97 47.2475) (width 1) (layer "B.Cu") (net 8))
 (segment (start 133.9665 47.244) (end 130.556 47.244) (width 1) (layer "B.Cu") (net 8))
 (segment (start 133.9665 47.244) (end 133.97 47.2475) (width 0.3048) (layer "B.Cu") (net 8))
 (segment (start 139.065 62.435) (end 139.065 67.94) (width 0.3048) (layer "B.Cu") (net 7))
 (segment (start 137.16 69.845) (end 137.16 71.12) (width 0.3048) (layer "B.Cu") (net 7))
 (segment (start 139.065 67.94) (end 137.16 69.845) (width 0.3048) (layer "B.Cu") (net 7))
 (segment (start 137.795 66.71) (end 134.62 69.885) (width 0.3048) (layer "B.Cu") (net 5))
 (segment (start 134.62 69.885) (end 134.62 71.12) (width 0.3048) (layer "B.Cu") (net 5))
 (segment (start 137.795 62.435) (end 137.795 66.71) (width 0.3048) (layer "B.Cu") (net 5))
 (segment (start 136.525 65.23) (end 132.08 69.675) (width 0.3048) (layer "B.Cu") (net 9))
 (segment (start 132.08 69.675) (end 132.08 71.12) (width 0.3048) (layer "B.Cu") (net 9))
 (segment (start 136.525 62.435) (end 136.525 65.23) (width 0.3048) (layer "B.Cu") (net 9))
 (segment (start 139.7 71.12) (end 139.7 69.6785) (width 0.3048) (layer "B.Cu") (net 10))
 (segment (start 141.605 67.7735) (end 141.605 62.435) (width 0.3048) (layer "B.Cu") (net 10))
 (segment (start 139.7 69.6785) (end 141.605 67.7735) (width 0.3048) (layer "B.Cu") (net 10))
 (segment (start 142.875 69.2655) (end 142.875 62.435) (width 0.3048) (layer "B.Cu") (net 2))
 (segment (start 142.24 69.9005) (end 142.875 69.2655) (width 0.3048) (layer "B.Cu") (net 2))
 (segment (start 142.24 71.12) (end 142.24 69.9005) (width 0.3048) (layer "B.Cu") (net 2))
 (segment (start 144.78 69.785) (end 144.145 69.15) (width 0.3048) (layer "B.Cu") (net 6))
 (segment (start 144.145 69.15) (end 144.145 62.435) (width 0.3048) (layer "B.Cu") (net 6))
 (segment (start 144.78 71.12) (end 144.78 69.785) (width 0.3048) (layer "B.Cu") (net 6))
 (segment (start 147.32 71.12) (end 147.32 69.7145) (width 0.3048) (layer "B.Cu") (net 4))
 (segment (start 147.32 69.7145) (end 145.415 67.8095) (width 0.3048) (layer "B.Cu") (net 4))
 (segment (start 145.415 67.8095) (end 145.415 62.435) (width 0.3048) (layer "B.Cu") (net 4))
 (segment (start 149.86 71.12) (end 149.86 69.6155) (width 0.3048) (layer "B.Cu") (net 1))
 (segment (start 149.86 69.6155) (end 146.685 66.4405) (width 0.3048) (layer "B.Cu") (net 1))
 (segment (start 146.685 66.4405) (end 146.685 62.435) (width 0.3048) (layer "B.Cu") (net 1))
 (segment (start 134.7875 56.2175) (end 136.47 54.535) (width 0.3048) (layer "B.Cu") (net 23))
 (segment (start 131.76 56.2175) (end 134.7875 56.2175) (width 0.3048) (layer "B.Cu") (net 23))
 (segment (start 136.525 53.135) (end 136.525 54.483) (width 0.3048) (layer "B.Cu") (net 23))
 (segment (start 136.525 54.483) (end 136.0955 54.9125) (width 0.3048) (layer "B.Cu") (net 23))
 (segment (start 150.02 55.485) (end 149.72 55.785) (width 0.3048) (layer "B.Cu") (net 22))
 (segment (start 150.02 54.3475) (end 150.02 55.485) (width 0.3048) (layer "B.Cu") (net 22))
 (segment (start 142.22 55.785) (end 141.605 55.17) (width 0.3048) (layer "B.Cu") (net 22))
 (segment (start 149.72 55.785) (end 142.22 55.785) (width 0.3048) (layer "B.Cu") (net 22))
 (segment (start 141.605 55.17) (end 141.605 53.135) (width 0.3048) (layer "B.Cu") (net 22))
 (segment (start 142.875 51.562) (end 140.247 51.562) (width 0.3048) (layer "F.Cu") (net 19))
 (segment (start 138.43 49.745) (end 138.43 48.285) (width 0.3048) (layer "F.Cu") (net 19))
 (segment (start 140.247 51.562) (end 138.43 49.745) (width 0.3048) (layer "F.Cu") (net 19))
 (via (at 142.875 51.562) (size 0.8) (drill 0.4) (layers "F.Cu" "B.Cu") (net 19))
 (segment (start 142.875 53.135) (end 142.875 51.562) (width 0.3048) (layer "B.Cu") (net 19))
 (segment (start 143.368 50.785) (end 141.97 50.785) (width 0.3048) (layer "F.Cu") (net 18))
 (segment (start 140.97 49.785) (end 140.97 48.285) (width 0.3048) (layer "F.Cu") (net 18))
 (segment (start 144.145 51.562) (end 143.368 50.785) (width 0.3048) (layer "F.Cu") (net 18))
 (segment (start 141.97 50.785) (end 140.97 49.785) (width 0.3048) (layer "F.Cu") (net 18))
 (via (at 144.145 51.562) (size 0.8) (drill 0.4) (layers "F.Cu" "B.Cu") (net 18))
 (segment (start 144.145 53.135) (end 144.145 51.562) (width 0.3048) (layer "B.Cu") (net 18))
 (segment (start 143.51 49.657) (end 145.415 51.562) (width 0.3048) (layer "F.Cu") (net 17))
 (segment (start 143.51 48.285) (end 143.51 49.325) (width 0.3048) (layer "F.Cu") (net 17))
 (segment (start 143.51 48.285) (end 143.51 49.657) (width 0.3048) (layer "F.Cu") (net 17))
 (via (at 145.415 51.562) (size 0.8) (drill 0.4) (layers "F.Cu" "B.Cu") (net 17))
 (segment (start 145.415 53.135) (end 145.415 51.562) (width 0.3048) (layer "B.Cu") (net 17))
 (segment (start 145.97 50.847) (end 145.97 48.365) (width 0.3048) (layer "F.Cu") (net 16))
 (segment (start 146.685 51.562) (end 145.97 50.847) (width 0.3048) (layer "F.Cu") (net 16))
 (segment (start 145.97 48.365) (end 146.05 48.285) (width 0.3048) (layer "F.Cu") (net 16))
 (via (at 146.685 51.562) (size 0.8) (drill 0.4) (layers "F.Cu" "B.Cu") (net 16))
 (segment (start 146.685 53.135) (end 146.685 51.562) (width 0.3048) (layer "B.Cu") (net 16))
 (segment (start 143.51 67.285) (end 143.51 57.912) (width 0.3048) (layer "F.Cu") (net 14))
 (segment (start 143.51 57.912) (end 140.462 54.864) (width 0.3048) (layer "F.Cu") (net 14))
 (via (at 140.462 54.864) (size 0.8) (drill 0.4) (layers "F.Cu" "B.Cu") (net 14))
 (segment (start 140.335 53.135) (end 140.335 54.737) (width 0.3048) (layer "B.Cu") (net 14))
 (segment (start 140.335 54.737) (end 140.462 54.864) (width 0.3048) (layer "B.Cu") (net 14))
 (segment (start 139.192 54.864) (end 140.97 56.642) (width 0.3048) (layer "F.Cu") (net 13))
 (segment (start 140.97 56.642) (end 140.97 67.285) (width 0.3048) (layer "F.Cu") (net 13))
 (via (at 139.192 54.864) (size 0.8) (drill 0.4) (layers "F.Cu" "B.Cu") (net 13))
 (segment (start 139.065 53.135) (end 139.065 54.737) (width 0.3048) (layer "B.Cu") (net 13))
 (segment (start 139.065 54.737) (end 139.192 54.864) (width 0.3048) (layer "B.Cu") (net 13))
 (segment (start 135.89 56.388) (end 135.89 67.285) (width 0.3048) (layer "F.Cu") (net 11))
 (via (at 135.89 56.388) (size 0.8) (drill 0.4) (layers "F.Cu" "B.Cu") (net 11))
 (segment (start 137.795 54.483) (end 135.89 56.388) (width 0.3048) (layer "B.Cu") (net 11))
 (segment (start 137.795 53.135) (end 137.795 54.483) (width 0.3048) (layer "B.Cu") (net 11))
 (segment (start 140.335 60.15) (end 140.335 62.435) (width 0.3048) (layer "B.Cu") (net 21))
 (segment (start 139.22 59.035) (end 140.335 60.15) (width 0.3048) (layer "B.Cu") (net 21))
 (segment (start 137.97 59.035) (end 139.22 59.035) (width 0.3048) (layer "B.Cu") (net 21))
 (segment (start 131.945 59.035) (end 137.915 59.035) (width 0.3048) (layer "B.Cu") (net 21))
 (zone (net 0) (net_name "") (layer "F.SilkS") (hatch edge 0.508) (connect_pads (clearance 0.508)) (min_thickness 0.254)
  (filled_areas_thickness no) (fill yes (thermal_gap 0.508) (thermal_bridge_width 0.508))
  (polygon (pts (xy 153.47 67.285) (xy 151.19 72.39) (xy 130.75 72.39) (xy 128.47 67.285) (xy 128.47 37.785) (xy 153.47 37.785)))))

